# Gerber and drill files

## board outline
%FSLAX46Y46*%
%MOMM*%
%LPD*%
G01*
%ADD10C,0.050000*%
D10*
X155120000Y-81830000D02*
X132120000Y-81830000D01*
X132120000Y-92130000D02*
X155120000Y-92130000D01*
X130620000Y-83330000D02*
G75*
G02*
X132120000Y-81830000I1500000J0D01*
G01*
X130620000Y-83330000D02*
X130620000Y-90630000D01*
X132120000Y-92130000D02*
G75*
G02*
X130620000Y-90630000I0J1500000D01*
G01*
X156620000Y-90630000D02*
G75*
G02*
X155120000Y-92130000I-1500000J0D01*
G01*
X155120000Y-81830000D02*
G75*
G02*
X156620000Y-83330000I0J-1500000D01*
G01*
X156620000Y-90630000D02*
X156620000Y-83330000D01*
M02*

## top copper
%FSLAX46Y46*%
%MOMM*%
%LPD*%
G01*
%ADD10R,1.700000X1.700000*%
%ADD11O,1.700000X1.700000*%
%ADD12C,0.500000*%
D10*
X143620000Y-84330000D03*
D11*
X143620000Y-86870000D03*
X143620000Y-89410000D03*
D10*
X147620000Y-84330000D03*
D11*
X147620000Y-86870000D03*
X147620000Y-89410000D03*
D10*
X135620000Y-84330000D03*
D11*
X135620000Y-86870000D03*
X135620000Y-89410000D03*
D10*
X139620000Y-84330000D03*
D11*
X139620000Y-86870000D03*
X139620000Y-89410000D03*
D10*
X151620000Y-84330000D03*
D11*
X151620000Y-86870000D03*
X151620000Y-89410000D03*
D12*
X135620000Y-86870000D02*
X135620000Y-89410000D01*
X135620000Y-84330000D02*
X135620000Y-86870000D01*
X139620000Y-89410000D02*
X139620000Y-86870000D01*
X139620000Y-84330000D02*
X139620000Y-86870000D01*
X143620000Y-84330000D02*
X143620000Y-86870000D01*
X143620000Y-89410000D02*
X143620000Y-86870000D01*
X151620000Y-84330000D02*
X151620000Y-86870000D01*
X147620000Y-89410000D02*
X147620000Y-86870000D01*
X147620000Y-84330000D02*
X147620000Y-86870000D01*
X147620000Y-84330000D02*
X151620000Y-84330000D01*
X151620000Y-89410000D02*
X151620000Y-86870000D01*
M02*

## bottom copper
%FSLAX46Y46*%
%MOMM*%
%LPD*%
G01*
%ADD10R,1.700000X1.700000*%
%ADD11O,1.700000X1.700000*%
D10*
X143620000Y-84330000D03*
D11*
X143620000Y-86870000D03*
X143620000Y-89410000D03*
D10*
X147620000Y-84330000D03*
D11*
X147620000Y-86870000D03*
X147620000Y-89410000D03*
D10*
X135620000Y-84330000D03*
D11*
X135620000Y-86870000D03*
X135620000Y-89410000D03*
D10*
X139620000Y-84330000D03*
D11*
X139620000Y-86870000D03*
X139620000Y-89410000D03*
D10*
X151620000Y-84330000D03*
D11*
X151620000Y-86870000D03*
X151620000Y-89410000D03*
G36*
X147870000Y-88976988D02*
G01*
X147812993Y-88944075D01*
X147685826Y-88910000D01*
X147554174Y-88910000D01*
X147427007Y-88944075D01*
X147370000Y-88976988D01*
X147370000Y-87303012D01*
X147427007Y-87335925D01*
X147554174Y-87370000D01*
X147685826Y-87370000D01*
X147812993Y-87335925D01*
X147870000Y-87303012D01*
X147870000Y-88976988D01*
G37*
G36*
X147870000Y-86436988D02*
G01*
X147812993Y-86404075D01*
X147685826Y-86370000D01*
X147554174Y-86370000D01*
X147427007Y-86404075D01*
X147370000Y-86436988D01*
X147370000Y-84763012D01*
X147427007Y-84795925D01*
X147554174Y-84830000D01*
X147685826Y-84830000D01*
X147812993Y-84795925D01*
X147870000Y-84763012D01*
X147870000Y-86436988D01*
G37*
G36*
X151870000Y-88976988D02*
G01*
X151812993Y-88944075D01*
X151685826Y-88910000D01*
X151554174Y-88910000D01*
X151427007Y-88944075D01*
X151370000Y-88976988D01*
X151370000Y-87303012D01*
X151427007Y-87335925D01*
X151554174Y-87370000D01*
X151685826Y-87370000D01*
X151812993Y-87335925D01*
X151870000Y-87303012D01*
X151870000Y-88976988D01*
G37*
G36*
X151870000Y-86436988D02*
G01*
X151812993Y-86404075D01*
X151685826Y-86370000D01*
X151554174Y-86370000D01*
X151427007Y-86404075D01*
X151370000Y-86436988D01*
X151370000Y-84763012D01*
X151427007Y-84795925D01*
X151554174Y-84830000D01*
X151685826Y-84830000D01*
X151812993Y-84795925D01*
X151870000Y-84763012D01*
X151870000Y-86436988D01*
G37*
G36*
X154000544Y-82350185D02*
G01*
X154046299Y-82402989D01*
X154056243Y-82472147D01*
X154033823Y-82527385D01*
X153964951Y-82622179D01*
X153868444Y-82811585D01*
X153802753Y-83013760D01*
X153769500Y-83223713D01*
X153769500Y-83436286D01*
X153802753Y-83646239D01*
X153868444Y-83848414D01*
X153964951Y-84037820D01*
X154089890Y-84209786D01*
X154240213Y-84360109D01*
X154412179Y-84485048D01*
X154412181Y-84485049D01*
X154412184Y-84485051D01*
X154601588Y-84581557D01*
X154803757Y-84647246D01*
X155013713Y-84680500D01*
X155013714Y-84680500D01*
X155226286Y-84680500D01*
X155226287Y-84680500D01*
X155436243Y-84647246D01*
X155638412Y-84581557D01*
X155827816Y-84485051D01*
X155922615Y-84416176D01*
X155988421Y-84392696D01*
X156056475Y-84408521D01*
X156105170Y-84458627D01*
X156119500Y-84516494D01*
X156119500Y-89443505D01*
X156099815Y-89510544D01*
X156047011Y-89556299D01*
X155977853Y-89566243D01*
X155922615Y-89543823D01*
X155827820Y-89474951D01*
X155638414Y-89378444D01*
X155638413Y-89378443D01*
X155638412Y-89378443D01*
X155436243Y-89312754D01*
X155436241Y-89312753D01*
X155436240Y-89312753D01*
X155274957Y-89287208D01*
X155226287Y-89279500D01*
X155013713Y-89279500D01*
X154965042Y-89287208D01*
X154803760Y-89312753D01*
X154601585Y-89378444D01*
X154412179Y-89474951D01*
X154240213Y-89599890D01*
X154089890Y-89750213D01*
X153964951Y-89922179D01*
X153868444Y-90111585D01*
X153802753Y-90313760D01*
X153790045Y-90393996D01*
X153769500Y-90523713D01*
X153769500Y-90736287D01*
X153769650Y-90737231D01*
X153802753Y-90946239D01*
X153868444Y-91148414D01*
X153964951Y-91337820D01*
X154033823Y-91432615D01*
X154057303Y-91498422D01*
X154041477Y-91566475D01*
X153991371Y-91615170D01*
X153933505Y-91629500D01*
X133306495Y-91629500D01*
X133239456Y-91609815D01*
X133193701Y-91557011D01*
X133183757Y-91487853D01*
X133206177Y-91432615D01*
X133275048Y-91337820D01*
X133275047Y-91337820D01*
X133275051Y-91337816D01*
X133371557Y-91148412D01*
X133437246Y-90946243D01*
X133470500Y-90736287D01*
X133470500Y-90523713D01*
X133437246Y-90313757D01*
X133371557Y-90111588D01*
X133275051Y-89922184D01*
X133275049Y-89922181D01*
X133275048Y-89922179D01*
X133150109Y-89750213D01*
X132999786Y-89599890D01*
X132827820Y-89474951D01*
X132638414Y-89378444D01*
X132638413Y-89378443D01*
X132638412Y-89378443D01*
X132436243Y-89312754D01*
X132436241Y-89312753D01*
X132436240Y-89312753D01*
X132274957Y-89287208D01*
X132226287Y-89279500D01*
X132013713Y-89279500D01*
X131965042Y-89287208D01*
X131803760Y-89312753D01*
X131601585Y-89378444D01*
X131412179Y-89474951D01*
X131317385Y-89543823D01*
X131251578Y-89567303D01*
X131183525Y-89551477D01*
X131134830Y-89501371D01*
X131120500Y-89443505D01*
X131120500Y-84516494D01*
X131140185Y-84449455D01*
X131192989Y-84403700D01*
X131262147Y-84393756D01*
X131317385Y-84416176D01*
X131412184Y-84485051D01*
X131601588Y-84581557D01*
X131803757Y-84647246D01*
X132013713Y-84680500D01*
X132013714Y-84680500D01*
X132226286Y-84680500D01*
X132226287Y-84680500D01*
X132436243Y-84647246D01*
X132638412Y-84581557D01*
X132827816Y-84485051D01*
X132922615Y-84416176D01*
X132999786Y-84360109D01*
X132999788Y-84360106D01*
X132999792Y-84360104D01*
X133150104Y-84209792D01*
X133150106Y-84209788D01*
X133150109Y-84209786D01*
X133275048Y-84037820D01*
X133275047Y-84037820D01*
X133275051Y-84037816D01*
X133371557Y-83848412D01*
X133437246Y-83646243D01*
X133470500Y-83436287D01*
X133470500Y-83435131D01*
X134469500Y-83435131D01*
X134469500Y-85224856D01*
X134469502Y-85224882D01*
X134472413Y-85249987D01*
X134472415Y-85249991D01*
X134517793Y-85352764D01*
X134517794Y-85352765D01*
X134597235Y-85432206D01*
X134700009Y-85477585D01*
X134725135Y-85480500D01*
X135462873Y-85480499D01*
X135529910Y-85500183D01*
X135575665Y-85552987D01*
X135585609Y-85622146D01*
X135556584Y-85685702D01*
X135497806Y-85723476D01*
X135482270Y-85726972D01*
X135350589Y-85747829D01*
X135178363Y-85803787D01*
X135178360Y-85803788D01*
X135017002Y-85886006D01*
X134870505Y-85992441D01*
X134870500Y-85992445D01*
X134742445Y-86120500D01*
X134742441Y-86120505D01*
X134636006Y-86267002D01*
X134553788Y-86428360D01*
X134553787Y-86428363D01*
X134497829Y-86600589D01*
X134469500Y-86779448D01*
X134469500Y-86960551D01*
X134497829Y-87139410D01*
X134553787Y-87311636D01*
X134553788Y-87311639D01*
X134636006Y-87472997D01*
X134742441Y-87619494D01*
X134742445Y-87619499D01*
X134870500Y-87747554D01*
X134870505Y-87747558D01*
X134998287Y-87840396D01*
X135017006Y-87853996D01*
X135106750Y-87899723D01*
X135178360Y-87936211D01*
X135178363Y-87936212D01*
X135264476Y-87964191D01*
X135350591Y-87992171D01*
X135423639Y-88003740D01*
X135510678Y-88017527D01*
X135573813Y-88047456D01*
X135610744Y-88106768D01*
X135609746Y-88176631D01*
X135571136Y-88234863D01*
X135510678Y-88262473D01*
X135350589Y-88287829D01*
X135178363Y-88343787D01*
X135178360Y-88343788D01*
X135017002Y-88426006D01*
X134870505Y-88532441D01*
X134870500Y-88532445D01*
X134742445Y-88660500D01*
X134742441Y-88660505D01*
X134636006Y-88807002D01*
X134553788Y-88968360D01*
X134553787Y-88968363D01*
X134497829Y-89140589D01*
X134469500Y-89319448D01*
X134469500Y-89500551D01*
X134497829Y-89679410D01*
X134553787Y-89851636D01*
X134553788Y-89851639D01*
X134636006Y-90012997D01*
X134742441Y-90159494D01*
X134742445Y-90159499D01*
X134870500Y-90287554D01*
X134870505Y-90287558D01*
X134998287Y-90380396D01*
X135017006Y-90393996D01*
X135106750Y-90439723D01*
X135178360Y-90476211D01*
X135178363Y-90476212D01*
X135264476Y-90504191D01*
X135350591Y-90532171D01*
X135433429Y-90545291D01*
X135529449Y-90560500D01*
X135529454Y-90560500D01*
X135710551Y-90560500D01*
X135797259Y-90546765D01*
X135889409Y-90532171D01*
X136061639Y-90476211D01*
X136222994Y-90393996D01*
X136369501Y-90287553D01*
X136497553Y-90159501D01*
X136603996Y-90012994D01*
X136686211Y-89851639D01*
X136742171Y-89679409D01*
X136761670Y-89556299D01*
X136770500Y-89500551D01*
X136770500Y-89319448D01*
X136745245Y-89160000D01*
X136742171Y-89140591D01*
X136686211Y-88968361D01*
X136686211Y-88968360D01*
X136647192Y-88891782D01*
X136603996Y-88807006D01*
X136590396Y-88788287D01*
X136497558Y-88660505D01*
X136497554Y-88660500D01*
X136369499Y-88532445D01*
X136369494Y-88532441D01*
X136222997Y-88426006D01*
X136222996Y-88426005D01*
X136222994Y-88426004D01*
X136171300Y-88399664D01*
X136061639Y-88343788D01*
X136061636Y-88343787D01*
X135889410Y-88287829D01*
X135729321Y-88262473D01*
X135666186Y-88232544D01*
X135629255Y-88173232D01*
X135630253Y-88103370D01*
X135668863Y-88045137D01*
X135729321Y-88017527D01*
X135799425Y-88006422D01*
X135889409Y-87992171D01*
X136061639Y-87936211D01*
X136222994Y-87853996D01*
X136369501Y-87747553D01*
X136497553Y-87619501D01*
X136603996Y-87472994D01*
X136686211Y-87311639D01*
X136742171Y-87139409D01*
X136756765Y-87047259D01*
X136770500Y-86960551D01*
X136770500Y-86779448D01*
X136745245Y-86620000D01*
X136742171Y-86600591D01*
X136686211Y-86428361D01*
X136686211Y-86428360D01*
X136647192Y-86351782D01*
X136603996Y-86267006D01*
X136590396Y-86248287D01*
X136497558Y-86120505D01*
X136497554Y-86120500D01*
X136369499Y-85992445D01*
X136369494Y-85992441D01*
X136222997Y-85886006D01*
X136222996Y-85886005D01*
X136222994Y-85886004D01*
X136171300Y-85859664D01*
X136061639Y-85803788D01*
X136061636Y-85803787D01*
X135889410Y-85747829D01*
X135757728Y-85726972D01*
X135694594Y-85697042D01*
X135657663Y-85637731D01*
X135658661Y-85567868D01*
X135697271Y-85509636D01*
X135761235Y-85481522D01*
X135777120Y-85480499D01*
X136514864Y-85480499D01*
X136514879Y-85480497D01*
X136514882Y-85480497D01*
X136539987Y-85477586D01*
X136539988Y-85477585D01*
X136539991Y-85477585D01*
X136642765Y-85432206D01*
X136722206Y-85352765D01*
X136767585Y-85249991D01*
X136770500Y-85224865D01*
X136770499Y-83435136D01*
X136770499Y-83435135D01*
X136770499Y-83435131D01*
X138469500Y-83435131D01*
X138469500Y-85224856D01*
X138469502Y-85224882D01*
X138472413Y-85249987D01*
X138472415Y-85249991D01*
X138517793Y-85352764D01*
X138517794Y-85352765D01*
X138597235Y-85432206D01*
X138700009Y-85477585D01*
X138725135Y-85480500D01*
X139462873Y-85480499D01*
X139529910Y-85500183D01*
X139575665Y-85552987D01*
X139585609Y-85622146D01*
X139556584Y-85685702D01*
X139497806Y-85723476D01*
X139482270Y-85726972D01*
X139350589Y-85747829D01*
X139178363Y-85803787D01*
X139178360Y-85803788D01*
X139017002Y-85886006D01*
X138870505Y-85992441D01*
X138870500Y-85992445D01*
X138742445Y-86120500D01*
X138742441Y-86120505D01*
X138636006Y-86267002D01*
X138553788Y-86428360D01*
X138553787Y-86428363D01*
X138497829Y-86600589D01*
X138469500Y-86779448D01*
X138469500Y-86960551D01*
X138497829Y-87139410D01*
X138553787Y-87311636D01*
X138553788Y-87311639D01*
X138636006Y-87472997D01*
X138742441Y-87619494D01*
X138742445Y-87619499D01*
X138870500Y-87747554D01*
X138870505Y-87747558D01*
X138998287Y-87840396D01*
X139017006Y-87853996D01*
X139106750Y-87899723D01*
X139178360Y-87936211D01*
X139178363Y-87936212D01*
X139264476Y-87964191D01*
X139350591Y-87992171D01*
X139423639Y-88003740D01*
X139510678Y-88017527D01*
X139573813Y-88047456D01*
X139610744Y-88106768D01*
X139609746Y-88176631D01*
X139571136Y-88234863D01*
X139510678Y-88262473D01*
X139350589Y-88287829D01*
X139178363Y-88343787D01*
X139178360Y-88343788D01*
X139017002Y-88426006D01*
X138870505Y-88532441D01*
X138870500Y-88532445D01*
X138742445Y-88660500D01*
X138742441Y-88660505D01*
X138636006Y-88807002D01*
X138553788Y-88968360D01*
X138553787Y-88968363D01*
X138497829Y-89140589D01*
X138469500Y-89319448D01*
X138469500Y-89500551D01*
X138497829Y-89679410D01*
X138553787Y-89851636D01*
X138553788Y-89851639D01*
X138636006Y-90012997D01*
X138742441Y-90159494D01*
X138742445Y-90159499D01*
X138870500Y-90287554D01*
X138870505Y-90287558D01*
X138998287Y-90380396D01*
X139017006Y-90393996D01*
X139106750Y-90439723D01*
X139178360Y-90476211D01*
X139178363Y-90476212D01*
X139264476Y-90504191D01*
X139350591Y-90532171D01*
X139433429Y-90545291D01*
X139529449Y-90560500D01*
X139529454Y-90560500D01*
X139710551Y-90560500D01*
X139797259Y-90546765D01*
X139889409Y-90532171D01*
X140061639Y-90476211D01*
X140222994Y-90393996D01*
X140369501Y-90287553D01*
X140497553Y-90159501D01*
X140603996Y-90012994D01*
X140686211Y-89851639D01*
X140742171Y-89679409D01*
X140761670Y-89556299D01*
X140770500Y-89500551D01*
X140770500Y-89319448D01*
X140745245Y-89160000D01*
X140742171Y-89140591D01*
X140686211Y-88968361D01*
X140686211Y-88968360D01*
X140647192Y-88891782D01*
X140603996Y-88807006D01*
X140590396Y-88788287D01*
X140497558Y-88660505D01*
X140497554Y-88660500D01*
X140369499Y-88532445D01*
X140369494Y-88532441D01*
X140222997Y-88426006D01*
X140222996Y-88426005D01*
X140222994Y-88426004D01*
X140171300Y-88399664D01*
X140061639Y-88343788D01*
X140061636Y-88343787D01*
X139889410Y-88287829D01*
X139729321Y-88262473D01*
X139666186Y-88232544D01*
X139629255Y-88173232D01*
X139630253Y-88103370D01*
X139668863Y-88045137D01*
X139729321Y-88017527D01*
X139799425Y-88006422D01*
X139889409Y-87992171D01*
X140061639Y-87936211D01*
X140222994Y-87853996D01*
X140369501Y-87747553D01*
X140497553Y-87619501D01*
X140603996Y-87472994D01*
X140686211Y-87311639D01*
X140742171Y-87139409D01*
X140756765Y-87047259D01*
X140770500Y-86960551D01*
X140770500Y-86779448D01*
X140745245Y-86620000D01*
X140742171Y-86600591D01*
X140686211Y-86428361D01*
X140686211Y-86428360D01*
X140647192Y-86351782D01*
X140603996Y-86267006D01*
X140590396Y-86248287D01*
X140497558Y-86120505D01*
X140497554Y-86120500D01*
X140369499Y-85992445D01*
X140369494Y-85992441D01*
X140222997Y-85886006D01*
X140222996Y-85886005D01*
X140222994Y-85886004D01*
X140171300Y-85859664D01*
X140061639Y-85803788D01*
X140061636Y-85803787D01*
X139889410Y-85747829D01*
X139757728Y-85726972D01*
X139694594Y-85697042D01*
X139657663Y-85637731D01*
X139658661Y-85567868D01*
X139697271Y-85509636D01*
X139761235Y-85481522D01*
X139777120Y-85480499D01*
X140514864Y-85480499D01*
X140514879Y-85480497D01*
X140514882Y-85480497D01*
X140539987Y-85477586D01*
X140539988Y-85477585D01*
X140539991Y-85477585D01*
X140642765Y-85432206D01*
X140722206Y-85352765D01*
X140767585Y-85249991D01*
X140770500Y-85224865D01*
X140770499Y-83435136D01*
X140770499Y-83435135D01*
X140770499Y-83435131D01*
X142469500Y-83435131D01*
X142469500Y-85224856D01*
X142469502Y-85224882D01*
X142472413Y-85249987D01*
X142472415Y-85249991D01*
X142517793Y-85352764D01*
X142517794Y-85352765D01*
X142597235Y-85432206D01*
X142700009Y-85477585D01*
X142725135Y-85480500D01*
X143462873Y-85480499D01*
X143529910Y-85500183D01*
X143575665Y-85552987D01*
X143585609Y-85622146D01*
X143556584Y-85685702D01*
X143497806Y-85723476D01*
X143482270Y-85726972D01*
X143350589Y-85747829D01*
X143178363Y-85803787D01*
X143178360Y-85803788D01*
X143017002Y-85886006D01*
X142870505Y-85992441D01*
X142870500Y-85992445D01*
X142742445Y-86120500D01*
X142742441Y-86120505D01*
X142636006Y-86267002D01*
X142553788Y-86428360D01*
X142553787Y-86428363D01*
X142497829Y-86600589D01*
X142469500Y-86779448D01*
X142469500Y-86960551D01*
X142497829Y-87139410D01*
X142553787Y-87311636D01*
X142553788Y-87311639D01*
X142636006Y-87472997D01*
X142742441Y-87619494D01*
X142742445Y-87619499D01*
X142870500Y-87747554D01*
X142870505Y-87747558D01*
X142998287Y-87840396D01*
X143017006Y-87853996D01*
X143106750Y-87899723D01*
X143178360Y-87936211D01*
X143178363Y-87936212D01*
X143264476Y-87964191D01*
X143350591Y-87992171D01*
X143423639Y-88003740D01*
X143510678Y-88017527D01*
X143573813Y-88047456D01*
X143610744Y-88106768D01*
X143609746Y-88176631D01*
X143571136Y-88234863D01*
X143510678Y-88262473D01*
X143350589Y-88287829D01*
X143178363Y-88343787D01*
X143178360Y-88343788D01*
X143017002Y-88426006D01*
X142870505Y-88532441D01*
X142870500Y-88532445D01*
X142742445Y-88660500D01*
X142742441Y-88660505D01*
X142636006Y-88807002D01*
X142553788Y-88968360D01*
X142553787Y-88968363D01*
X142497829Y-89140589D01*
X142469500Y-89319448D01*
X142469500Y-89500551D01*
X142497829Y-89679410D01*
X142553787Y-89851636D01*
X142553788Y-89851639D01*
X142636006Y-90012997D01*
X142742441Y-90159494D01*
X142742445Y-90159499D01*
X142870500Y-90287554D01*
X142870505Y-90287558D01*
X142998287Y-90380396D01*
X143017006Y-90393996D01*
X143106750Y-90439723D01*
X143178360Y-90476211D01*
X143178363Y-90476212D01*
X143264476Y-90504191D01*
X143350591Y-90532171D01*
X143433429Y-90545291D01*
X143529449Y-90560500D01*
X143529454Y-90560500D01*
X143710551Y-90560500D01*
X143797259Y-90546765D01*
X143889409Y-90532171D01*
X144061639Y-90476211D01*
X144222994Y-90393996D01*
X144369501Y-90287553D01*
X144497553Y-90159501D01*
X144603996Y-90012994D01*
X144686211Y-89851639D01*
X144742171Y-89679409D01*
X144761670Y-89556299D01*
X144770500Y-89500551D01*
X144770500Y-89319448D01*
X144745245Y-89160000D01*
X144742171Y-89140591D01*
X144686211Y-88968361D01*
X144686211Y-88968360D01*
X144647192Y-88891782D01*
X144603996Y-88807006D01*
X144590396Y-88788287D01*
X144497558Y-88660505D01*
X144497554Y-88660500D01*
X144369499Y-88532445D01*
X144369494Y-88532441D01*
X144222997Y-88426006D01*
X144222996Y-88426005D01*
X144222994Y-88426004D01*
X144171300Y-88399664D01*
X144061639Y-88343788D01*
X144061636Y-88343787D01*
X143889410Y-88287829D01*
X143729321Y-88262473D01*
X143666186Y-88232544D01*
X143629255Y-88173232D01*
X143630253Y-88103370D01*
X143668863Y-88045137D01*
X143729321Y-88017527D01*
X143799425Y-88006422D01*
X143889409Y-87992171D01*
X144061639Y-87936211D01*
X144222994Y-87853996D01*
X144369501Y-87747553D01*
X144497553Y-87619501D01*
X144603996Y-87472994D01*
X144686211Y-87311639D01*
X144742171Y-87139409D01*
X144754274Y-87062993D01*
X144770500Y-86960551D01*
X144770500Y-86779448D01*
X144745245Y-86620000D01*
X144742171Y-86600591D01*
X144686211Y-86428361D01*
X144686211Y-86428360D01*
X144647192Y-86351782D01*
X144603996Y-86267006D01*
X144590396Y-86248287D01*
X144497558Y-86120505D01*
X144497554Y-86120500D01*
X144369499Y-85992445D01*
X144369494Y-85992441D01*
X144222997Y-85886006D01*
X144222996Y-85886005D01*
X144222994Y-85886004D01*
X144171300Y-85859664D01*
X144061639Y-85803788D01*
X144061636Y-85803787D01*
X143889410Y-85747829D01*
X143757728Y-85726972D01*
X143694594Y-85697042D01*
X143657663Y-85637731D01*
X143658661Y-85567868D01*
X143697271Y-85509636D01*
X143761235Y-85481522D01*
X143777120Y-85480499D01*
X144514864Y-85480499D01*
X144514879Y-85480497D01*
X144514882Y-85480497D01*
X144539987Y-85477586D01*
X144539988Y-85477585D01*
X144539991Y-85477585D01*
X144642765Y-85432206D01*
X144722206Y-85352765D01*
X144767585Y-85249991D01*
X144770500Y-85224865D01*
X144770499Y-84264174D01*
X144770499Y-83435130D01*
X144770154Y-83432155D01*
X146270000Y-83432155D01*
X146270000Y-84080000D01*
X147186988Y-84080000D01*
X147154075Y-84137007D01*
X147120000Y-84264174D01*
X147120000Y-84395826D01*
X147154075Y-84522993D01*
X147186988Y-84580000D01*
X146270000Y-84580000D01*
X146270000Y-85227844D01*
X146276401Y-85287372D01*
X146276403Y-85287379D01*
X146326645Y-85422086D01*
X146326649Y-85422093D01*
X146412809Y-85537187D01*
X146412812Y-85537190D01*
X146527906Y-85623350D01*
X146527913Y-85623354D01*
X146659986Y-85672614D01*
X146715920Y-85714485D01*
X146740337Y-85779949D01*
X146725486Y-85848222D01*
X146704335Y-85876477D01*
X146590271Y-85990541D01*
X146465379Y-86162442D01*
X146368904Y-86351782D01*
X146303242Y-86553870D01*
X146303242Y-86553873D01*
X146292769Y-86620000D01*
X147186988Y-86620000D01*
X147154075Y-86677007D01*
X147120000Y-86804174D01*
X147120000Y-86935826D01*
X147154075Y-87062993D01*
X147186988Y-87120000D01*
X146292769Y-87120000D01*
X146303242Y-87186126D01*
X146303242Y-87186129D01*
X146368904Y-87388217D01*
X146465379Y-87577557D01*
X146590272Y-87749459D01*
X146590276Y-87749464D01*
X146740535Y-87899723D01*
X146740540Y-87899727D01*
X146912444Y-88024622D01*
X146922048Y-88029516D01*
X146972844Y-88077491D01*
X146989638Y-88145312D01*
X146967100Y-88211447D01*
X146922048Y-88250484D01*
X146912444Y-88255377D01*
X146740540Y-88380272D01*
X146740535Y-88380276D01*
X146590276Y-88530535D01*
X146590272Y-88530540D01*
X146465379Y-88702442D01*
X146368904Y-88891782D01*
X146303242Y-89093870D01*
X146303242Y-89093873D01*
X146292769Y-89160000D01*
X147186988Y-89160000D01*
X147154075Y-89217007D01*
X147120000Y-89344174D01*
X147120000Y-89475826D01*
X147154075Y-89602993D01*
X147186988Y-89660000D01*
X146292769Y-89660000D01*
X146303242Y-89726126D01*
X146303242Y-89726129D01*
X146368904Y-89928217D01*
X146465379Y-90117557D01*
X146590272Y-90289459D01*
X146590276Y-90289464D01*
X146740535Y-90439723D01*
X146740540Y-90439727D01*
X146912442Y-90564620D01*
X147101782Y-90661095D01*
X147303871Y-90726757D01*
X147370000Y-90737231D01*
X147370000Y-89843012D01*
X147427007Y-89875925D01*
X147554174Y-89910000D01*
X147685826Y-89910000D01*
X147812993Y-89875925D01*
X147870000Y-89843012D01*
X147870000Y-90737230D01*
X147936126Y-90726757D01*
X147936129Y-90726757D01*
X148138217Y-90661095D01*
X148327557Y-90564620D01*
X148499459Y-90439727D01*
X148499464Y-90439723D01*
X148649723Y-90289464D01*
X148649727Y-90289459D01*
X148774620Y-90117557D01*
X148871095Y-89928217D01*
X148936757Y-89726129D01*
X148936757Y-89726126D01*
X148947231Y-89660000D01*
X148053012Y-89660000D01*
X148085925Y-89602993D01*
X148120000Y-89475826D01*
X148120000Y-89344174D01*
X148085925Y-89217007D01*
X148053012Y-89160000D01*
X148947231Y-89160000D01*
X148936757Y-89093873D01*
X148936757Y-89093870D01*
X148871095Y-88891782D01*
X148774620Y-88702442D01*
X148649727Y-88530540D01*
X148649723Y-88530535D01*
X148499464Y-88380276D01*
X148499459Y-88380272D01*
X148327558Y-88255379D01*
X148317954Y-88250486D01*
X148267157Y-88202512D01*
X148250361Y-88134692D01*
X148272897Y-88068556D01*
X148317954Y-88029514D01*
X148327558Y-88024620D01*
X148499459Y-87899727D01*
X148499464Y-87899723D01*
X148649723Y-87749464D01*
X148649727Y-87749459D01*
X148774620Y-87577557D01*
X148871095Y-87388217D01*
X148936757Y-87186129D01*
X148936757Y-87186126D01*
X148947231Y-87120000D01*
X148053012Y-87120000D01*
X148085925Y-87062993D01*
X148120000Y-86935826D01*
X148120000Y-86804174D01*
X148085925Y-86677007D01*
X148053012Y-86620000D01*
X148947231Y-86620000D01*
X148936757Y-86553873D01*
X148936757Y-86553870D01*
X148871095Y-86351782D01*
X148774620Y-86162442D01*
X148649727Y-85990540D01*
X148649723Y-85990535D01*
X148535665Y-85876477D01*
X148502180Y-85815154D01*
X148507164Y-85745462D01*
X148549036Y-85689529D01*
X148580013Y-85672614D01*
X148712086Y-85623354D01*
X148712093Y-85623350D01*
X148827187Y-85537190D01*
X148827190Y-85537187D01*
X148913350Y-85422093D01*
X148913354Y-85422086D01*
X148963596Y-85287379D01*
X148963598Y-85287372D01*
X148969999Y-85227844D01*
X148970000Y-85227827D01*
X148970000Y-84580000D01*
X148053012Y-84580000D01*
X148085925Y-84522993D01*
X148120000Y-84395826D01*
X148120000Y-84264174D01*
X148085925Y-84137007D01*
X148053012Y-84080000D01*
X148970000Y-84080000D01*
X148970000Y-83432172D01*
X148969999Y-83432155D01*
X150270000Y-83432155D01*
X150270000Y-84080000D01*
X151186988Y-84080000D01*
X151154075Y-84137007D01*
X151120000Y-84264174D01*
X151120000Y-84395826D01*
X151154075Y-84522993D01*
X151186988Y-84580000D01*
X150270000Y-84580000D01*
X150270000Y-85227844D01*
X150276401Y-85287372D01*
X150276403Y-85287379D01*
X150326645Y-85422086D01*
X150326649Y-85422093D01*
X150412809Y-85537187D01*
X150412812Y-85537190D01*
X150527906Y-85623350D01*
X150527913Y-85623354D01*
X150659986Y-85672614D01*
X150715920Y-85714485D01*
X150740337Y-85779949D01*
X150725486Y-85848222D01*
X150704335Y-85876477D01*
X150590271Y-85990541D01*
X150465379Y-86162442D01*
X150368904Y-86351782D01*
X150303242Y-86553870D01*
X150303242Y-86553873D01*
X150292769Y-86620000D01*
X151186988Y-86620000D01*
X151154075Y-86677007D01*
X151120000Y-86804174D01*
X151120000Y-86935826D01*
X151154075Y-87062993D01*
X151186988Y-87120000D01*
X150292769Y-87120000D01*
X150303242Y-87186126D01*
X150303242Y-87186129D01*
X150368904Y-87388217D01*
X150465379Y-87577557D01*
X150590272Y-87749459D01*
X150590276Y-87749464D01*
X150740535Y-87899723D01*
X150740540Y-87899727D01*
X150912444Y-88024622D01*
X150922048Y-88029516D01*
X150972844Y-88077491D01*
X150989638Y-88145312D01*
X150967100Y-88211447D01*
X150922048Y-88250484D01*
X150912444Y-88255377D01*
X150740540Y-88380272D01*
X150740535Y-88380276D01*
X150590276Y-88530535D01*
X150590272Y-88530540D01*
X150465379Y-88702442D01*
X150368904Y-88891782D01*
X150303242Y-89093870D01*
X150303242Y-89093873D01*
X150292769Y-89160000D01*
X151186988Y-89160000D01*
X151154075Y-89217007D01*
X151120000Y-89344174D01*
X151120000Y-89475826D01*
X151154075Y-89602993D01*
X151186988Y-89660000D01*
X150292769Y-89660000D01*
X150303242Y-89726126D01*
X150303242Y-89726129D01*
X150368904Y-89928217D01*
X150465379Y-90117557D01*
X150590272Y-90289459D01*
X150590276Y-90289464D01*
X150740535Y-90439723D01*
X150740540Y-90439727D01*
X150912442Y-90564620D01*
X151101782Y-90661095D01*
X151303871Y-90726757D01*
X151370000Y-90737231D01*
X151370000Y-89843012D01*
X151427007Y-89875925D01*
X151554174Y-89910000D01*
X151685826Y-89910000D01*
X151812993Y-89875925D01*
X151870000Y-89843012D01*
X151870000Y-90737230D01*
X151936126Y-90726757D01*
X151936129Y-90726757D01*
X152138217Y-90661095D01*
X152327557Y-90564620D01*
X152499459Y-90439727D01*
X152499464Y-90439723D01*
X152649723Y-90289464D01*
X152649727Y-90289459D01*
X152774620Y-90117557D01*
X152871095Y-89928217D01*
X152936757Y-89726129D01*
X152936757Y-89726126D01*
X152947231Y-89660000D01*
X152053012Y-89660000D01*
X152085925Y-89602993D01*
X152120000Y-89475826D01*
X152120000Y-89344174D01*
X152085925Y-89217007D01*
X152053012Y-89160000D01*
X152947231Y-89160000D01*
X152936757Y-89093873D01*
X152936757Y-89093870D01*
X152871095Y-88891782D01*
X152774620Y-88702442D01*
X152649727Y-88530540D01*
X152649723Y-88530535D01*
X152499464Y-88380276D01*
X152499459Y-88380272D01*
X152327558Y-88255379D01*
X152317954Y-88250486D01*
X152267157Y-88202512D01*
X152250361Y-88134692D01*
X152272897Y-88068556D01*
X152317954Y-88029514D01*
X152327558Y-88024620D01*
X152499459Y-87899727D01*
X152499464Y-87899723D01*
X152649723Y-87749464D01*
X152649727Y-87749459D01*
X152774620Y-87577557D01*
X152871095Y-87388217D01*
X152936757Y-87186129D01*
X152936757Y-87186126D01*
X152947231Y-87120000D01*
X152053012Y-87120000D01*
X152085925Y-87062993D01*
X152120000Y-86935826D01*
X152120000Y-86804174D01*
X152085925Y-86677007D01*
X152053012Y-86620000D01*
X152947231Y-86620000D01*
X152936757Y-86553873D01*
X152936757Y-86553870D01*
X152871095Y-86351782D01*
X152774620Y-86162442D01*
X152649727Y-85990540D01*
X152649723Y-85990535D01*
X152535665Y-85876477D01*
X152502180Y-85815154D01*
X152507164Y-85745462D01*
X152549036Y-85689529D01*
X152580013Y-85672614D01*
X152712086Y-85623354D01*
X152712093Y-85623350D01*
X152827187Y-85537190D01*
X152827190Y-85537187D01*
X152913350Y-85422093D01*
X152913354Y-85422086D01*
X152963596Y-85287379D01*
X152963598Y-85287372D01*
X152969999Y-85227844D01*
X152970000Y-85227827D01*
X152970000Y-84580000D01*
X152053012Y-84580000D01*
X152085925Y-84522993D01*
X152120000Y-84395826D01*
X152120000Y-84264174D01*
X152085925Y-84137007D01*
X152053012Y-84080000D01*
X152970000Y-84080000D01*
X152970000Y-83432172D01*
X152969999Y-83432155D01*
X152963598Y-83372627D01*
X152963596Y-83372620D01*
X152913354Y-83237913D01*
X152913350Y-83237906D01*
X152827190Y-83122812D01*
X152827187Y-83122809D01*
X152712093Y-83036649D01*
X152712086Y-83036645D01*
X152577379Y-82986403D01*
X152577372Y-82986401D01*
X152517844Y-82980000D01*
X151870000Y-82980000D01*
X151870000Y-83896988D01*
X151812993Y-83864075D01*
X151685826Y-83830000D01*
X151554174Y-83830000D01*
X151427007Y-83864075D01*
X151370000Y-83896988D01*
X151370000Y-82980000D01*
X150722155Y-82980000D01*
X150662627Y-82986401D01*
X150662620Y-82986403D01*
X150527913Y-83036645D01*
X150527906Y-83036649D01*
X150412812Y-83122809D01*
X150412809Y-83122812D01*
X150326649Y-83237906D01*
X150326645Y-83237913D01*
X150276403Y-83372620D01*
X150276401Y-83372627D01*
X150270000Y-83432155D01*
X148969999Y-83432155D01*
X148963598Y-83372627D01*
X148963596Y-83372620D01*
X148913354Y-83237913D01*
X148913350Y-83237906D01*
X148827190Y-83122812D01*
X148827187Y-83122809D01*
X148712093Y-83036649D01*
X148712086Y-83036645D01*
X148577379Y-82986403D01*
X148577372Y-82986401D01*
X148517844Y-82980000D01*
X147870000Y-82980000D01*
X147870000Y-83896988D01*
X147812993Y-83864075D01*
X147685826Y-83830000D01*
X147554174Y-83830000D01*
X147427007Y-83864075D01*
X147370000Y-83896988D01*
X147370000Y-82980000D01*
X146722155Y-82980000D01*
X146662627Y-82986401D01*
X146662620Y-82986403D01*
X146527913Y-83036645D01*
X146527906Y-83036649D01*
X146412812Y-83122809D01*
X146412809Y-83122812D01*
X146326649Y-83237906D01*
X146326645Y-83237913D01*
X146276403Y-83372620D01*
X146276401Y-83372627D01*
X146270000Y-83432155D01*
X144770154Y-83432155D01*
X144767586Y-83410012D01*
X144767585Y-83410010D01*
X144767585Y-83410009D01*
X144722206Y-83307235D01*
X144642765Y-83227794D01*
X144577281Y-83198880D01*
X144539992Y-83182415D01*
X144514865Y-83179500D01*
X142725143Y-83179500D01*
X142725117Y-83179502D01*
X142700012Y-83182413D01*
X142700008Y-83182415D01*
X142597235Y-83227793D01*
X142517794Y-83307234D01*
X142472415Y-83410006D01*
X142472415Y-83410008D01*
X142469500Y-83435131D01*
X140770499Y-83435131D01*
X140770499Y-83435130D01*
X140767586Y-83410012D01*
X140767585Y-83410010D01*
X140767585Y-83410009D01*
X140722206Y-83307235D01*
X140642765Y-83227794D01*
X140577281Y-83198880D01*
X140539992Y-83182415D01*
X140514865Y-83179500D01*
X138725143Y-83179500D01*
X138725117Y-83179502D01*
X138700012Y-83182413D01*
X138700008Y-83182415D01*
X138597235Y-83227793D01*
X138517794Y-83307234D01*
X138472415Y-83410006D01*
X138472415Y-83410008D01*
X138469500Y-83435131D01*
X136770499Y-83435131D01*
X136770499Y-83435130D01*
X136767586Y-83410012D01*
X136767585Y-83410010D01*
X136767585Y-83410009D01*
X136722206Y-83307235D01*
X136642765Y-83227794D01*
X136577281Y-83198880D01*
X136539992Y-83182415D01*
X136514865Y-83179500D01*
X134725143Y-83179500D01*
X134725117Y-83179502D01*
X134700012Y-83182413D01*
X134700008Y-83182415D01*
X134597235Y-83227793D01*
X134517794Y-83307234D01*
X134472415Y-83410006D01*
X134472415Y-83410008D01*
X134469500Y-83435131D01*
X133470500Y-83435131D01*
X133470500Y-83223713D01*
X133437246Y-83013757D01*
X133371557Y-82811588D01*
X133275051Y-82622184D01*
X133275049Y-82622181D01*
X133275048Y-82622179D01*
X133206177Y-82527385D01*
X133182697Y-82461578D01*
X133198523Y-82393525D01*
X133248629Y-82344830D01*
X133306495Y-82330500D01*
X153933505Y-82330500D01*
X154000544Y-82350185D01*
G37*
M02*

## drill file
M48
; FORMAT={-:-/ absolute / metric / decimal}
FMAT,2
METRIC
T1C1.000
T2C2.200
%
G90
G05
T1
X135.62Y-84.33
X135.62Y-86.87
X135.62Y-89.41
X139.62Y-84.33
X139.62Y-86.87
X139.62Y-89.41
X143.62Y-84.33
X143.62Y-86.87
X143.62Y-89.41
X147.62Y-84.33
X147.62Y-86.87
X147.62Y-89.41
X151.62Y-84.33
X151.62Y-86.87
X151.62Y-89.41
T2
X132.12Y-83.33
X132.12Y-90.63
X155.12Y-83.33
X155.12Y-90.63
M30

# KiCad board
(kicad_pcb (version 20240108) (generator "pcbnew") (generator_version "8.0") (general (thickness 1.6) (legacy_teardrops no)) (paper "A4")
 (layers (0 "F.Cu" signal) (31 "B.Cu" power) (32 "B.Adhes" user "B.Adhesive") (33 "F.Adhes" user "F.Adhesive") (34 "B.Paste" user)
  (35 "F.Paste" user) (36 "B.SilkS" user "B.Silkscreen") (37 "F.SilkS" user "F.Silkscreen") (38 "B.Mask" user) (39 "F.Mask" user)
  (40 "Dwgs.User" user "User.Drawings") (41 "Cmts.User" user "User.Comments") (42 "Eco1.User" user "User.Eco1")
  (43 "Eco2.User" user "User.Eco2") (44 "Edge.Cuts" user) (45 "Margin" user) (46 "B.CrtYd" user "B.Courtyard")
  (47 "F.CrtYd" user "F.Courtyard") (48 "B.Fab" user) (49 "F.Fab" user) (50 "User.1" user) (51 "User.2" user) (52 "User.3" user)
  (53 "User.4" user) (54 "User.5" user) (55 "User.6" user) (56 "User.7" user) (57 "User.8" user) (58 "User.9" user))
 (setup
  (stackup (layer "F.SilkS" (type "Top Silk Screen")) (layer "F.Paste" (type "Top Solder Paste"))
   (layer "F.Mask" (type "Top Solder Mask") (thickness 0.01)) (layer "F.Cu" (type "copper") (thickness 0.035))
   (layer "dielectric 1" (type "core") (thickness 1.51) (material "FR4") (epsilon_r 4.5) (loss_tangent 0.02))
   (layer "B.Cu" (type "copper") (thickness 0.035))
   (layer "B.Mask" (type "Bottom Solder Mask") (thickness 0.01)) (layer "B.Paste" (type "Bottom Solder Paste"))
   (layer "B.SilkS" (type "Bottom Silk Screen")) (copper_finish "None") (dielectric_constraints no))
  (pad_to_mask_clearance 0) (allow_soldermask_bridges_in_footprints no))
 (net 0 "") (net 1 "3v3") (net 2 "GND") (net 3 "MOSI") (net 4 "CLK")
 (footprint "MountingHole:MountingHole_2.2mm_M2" (layer "F.Cu") (at 132.12 90.63)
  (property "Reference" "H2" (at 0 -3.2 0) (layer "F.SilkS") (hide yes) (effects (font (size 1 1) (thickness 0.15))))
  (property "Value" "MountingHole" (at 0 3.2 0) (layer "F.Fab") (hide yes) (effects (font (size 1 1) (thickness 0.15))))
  (pad "" np_thru_hole circle (at 0 0) (size 2.2 2.2) (drill 2.2) (layers "*.Cu" "*.Mask")))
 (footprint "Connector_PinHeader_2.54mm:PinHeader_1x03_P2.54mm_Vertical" (layer "F.Cu") (at 143.62 84.33)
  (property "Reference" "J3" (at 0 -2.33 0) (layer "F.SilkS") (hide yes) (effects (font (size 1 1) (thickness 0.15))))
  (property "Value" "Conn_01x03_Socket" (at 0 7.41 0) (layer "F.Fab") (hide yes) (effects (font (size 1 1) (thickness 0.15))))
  (pad "1" thru_hole rect (at 0 0) (size 1.7 1.7) (drill 1) (layers "*.Cu" "*.Mask") (remove_unused_layers no) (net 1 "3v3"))
  (pad "2" thru_hole oval (at 0 2.54) (size 1.7 1.7) (drill 1) (layers "*.Cu" "*.Mask") (remove_unused_layers no) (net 1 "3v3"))
  (pad "3" thru_hole oval (at 0 5.08) (size 1.7 1.7) (drill 1) (layers "*.Cu" "*.Mask") (remove_unused_layers no) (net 1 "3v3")))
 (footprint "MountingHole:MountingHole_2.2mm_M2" (layer "F.Cu") (at 155.12 83.33)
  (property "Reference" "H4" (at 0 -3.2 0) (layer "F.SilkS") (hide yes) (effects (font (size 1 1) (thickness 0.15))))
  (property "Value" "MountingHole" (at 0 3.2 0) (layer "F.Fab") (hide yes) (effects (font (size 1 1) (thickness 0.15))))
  (pad "" np_thru_hole circle (at 0 0) (size 2.2 2.2) (drill 2.2) (layers "*.Cu" "*.Mask")))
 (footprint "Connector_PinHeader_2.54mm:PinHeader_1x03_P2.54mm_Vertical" (layer "F.Cu") (at 147.62 84.33)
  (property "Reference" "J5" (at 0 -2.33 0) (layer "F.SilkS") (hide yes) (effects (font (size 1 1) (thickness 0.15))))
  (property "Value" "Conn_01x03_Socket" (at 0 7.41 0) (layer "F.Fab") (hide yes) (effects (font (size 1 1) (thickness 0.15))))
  (pad "1" thru_hole rect (at 0 0) (size 1.7 1.7) (drill 1) (layers "*.Cu" "*.Mask") (remove_unused_layers no) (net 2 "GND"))
  (pad "2" thru_hole oval (at 0 2.54) (size 1.7 1.7) (drill 1) (layers "*.Cu" "*.Mask") (remove_unused_layers no) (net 2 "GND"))
  (pad "3" thru_hole oval (at 0 5.08) (size 1.7 1.7) (drill 1) (layers "*.Cu" "*.Mask") (remove_unused_layers no) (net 2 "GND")))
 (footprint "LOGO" (layer "F.Cu") (at 132.46 87.06 90)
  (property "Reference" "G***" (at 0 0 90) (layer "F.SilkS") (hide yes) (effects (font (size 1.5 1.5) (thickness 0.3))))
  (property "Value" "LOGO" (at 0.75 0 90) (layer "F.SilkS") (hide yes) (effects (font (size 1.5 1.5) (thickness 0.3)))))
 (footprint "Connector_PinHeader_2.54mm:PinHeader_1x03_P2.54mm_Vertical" (layer "F.Cu") (at 135.62 84.33)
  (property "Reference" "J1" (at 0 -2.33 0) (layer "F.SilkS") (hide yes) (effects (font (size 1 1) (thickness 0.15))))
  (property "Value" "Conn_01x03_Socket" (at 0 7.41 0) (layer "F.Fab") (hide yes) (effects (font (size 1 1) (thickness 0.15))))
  (pad "1" thru_hole rect (at 0 0) (size 1.7 1.7) (drill 1) (layers "*.Cu" "*.Mask") (remove_unused_layers no) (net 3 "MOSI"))
  (pad "2" thru_hole oval (at 0 2.54) (size 1.7 1.7) (drill 1) (layers "*.Cu" "*.Mask") (remove_unused_layers no) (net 3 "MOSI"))
  (pad "3" thru_hole oval (at 0 5.08) (size 1.7 1.7) (drill 1) (layers "*.Cu" "*.Mask") (remove_unused_layers no) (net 3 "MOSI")))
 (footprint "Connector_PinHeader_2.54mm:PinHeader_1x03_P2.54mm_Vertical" (layer "F.Cu") (at 139.62 84.33)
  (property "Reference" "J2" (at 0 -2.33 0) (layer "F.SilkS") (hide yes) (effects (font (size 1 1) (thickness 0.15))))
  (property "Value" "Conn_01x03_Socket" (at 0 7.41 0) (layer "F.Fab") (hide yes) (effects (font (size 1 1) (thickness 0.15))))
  (pad "1" thru_hole rect (at 0 0) (size 1.7 1.7) (drill 1) (layers "*.Cu" "*.Mask") (remove_unused_layers no) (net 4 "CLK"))
  (pad "2" thru_hole oval (at 0 2.54) (size 1.7 1.7) (drill 1) (layers "*.Cu" "*.Mask") (remove_unused_layers no) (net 4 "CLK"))
  (pad "3" thru_hole oval (at 0 5.08) (size 1.7 1.7) (drill 1) (layers "*.Cu" "*.Mask") (remove_unused_layers no) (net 4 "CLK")))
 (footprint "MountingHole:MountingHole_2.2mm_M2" (layer "F.Cu") (at 155.12 90.63)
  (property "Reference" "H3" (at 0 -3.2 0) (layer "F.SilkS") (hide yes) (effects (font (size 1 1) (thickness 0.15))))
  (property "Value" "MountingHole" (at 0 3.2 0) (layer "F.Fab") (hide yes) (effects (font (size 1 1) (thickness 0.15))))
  (pad "" np_thru_hole circle (at 0 0) (size 2.2 2.2) (drill 2.2) (layers "*.Cu" "*.Mask")))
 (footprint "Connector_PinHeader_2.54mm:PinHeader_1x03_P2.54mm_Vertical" (layer "F.Cu") (at 151.62 84.33)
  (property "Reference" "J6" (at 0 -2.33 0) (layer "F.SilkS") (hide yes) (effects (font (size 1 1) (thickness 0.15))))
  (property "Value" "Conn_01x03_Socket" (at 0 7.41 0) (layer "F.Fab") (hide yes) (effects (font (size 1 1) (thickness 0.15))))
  (pad "1" thru_hole rect (at 0 0) (size 1.7 1.7) (drill 1) (layers "*.Cu" "*.Mask") (remove_unused_layers no) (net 2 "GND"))
  (pad "2" thru_hole oval (at 0 2.54) (size 1.7 1.7) (drill 1) (layers "*.Cu" "*.Mask") (remove_unused_layers no) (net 2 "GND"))
  (pad "3" thru_hole oval (at 0 5.08) (size 1.7 1.7) (drill 1) (layers "*.Cu" "*.Mask") (remove_unused_layers no) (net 2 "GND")))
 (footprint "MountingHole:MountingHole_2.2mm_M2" (layer "F.Cu") (at 132.12 83.33)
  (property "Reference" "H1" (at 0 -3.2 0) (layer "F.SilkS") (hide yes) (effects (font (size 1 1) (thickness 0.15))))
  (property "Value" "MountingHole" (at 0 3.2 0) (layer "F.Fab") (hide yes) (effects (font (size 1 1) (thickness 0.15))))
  (pad "" np_thru_hole circle (at 0 0) (size 2.2 2.2) (drill 2.2) (layers "*.Cu" "*.Mask")))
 (gr_line (start 155.12 81.83) (end 132.12 81.83) (stroke (width 0.05) (type default)) (layer "Edge.Cuts"))
 (gr_line (start 132.12 92.13) (end 155.12 92.13) (stroke (width 0.05) (type default)) (layer "Edge.Cuts"))
 (gr_arc (start 130.62 83.33) (mid 131.05934 82.26934) (end 132.12 81.83) (stroke (width 0.05) (type default)) (layer "Edge.Cuts"))
 (gr_line (start 130.62 83.33) (end 130.62 90.63) (stroke (width 0.05) (type default)) (layer "Edge.Cuts"))
 (gr_arc (start 132.12 92.13) (mid 131.05934 91.69066) (end 130.62 90.63) (stroke (width 0.05) (type default)) (layer "Edge.Cuts"))
 (gr_arc (start 156.62 90.63) (mid 156.18066 91.69066) (end 155.12 92.13) (stroke (width 0.05) (type default)) (layer "Edge.Cuts"))
 (gr_arc (start 155.12 81.83) (mid 156.18066 82.26934) (end 156.62 83.33) (stroke (width 0.05) (type default)) (layer "Edge.Cuts"))
 (gr_line (start 156.62 90.63) (end 156.62 83.33) (stroke (width 0.05) (type default)) (layer "Edge.Cuts"))
 (segment (start 135.62 86.87) (end 135.62 89.41) (width 0.5) (layer "F.Cu") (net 3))
 (segment (start 135.62 84.33) (end 135.62 86.87) (width 0.5) (layer "F.Cu") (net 3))
 (segment (start 139.62 89.41) (end 139.62 86.87) (width 0.5) (layer "F.Cu") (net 4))
 (segment (start 139.62 84.33) (end 139.62 86.87) (width 0.5) (layer "F.Cu") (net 4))
 (segment (start 143.62 84.33) (end 143.62 86.87) (width 0.5) (layer "F.Cu") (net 1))
 (segment (start 143.62 89.41) (end 143.62 86.87) (width 0.5) (layer "F.Cu") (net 1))
 (segment (start 151.62 84.33) (end 151.62 86.87) (width 0.5) (layer "F.Cu") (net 2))
 (segment (start 147.62 89.41) (end 147.62 86.87) (width 0.5) (layer "F.Cu") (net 2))
 (segment (start 147.62 84.33) (end 147.62 86.87) (width 0.5) (layer "F.Cu") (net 2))
 (segment (start 147.62 84.33) (end 151.62 84.33) (width 0.5) (layer "F.Cu") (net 2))
 (segment (start 151.62 89.41) (end 151.62 86.87) (width 0.5) (layer "F.Cu") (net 2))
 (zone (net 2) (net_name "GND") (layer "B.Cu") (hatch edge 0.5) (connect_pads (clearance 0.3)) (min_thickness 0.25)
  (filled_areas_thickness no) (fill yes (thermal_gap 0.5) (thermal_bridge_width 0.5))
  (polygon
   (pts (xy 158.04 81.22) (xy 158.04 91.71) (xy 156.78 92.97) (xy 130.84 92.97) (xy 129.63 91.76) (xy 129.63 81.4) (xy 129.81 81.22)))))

